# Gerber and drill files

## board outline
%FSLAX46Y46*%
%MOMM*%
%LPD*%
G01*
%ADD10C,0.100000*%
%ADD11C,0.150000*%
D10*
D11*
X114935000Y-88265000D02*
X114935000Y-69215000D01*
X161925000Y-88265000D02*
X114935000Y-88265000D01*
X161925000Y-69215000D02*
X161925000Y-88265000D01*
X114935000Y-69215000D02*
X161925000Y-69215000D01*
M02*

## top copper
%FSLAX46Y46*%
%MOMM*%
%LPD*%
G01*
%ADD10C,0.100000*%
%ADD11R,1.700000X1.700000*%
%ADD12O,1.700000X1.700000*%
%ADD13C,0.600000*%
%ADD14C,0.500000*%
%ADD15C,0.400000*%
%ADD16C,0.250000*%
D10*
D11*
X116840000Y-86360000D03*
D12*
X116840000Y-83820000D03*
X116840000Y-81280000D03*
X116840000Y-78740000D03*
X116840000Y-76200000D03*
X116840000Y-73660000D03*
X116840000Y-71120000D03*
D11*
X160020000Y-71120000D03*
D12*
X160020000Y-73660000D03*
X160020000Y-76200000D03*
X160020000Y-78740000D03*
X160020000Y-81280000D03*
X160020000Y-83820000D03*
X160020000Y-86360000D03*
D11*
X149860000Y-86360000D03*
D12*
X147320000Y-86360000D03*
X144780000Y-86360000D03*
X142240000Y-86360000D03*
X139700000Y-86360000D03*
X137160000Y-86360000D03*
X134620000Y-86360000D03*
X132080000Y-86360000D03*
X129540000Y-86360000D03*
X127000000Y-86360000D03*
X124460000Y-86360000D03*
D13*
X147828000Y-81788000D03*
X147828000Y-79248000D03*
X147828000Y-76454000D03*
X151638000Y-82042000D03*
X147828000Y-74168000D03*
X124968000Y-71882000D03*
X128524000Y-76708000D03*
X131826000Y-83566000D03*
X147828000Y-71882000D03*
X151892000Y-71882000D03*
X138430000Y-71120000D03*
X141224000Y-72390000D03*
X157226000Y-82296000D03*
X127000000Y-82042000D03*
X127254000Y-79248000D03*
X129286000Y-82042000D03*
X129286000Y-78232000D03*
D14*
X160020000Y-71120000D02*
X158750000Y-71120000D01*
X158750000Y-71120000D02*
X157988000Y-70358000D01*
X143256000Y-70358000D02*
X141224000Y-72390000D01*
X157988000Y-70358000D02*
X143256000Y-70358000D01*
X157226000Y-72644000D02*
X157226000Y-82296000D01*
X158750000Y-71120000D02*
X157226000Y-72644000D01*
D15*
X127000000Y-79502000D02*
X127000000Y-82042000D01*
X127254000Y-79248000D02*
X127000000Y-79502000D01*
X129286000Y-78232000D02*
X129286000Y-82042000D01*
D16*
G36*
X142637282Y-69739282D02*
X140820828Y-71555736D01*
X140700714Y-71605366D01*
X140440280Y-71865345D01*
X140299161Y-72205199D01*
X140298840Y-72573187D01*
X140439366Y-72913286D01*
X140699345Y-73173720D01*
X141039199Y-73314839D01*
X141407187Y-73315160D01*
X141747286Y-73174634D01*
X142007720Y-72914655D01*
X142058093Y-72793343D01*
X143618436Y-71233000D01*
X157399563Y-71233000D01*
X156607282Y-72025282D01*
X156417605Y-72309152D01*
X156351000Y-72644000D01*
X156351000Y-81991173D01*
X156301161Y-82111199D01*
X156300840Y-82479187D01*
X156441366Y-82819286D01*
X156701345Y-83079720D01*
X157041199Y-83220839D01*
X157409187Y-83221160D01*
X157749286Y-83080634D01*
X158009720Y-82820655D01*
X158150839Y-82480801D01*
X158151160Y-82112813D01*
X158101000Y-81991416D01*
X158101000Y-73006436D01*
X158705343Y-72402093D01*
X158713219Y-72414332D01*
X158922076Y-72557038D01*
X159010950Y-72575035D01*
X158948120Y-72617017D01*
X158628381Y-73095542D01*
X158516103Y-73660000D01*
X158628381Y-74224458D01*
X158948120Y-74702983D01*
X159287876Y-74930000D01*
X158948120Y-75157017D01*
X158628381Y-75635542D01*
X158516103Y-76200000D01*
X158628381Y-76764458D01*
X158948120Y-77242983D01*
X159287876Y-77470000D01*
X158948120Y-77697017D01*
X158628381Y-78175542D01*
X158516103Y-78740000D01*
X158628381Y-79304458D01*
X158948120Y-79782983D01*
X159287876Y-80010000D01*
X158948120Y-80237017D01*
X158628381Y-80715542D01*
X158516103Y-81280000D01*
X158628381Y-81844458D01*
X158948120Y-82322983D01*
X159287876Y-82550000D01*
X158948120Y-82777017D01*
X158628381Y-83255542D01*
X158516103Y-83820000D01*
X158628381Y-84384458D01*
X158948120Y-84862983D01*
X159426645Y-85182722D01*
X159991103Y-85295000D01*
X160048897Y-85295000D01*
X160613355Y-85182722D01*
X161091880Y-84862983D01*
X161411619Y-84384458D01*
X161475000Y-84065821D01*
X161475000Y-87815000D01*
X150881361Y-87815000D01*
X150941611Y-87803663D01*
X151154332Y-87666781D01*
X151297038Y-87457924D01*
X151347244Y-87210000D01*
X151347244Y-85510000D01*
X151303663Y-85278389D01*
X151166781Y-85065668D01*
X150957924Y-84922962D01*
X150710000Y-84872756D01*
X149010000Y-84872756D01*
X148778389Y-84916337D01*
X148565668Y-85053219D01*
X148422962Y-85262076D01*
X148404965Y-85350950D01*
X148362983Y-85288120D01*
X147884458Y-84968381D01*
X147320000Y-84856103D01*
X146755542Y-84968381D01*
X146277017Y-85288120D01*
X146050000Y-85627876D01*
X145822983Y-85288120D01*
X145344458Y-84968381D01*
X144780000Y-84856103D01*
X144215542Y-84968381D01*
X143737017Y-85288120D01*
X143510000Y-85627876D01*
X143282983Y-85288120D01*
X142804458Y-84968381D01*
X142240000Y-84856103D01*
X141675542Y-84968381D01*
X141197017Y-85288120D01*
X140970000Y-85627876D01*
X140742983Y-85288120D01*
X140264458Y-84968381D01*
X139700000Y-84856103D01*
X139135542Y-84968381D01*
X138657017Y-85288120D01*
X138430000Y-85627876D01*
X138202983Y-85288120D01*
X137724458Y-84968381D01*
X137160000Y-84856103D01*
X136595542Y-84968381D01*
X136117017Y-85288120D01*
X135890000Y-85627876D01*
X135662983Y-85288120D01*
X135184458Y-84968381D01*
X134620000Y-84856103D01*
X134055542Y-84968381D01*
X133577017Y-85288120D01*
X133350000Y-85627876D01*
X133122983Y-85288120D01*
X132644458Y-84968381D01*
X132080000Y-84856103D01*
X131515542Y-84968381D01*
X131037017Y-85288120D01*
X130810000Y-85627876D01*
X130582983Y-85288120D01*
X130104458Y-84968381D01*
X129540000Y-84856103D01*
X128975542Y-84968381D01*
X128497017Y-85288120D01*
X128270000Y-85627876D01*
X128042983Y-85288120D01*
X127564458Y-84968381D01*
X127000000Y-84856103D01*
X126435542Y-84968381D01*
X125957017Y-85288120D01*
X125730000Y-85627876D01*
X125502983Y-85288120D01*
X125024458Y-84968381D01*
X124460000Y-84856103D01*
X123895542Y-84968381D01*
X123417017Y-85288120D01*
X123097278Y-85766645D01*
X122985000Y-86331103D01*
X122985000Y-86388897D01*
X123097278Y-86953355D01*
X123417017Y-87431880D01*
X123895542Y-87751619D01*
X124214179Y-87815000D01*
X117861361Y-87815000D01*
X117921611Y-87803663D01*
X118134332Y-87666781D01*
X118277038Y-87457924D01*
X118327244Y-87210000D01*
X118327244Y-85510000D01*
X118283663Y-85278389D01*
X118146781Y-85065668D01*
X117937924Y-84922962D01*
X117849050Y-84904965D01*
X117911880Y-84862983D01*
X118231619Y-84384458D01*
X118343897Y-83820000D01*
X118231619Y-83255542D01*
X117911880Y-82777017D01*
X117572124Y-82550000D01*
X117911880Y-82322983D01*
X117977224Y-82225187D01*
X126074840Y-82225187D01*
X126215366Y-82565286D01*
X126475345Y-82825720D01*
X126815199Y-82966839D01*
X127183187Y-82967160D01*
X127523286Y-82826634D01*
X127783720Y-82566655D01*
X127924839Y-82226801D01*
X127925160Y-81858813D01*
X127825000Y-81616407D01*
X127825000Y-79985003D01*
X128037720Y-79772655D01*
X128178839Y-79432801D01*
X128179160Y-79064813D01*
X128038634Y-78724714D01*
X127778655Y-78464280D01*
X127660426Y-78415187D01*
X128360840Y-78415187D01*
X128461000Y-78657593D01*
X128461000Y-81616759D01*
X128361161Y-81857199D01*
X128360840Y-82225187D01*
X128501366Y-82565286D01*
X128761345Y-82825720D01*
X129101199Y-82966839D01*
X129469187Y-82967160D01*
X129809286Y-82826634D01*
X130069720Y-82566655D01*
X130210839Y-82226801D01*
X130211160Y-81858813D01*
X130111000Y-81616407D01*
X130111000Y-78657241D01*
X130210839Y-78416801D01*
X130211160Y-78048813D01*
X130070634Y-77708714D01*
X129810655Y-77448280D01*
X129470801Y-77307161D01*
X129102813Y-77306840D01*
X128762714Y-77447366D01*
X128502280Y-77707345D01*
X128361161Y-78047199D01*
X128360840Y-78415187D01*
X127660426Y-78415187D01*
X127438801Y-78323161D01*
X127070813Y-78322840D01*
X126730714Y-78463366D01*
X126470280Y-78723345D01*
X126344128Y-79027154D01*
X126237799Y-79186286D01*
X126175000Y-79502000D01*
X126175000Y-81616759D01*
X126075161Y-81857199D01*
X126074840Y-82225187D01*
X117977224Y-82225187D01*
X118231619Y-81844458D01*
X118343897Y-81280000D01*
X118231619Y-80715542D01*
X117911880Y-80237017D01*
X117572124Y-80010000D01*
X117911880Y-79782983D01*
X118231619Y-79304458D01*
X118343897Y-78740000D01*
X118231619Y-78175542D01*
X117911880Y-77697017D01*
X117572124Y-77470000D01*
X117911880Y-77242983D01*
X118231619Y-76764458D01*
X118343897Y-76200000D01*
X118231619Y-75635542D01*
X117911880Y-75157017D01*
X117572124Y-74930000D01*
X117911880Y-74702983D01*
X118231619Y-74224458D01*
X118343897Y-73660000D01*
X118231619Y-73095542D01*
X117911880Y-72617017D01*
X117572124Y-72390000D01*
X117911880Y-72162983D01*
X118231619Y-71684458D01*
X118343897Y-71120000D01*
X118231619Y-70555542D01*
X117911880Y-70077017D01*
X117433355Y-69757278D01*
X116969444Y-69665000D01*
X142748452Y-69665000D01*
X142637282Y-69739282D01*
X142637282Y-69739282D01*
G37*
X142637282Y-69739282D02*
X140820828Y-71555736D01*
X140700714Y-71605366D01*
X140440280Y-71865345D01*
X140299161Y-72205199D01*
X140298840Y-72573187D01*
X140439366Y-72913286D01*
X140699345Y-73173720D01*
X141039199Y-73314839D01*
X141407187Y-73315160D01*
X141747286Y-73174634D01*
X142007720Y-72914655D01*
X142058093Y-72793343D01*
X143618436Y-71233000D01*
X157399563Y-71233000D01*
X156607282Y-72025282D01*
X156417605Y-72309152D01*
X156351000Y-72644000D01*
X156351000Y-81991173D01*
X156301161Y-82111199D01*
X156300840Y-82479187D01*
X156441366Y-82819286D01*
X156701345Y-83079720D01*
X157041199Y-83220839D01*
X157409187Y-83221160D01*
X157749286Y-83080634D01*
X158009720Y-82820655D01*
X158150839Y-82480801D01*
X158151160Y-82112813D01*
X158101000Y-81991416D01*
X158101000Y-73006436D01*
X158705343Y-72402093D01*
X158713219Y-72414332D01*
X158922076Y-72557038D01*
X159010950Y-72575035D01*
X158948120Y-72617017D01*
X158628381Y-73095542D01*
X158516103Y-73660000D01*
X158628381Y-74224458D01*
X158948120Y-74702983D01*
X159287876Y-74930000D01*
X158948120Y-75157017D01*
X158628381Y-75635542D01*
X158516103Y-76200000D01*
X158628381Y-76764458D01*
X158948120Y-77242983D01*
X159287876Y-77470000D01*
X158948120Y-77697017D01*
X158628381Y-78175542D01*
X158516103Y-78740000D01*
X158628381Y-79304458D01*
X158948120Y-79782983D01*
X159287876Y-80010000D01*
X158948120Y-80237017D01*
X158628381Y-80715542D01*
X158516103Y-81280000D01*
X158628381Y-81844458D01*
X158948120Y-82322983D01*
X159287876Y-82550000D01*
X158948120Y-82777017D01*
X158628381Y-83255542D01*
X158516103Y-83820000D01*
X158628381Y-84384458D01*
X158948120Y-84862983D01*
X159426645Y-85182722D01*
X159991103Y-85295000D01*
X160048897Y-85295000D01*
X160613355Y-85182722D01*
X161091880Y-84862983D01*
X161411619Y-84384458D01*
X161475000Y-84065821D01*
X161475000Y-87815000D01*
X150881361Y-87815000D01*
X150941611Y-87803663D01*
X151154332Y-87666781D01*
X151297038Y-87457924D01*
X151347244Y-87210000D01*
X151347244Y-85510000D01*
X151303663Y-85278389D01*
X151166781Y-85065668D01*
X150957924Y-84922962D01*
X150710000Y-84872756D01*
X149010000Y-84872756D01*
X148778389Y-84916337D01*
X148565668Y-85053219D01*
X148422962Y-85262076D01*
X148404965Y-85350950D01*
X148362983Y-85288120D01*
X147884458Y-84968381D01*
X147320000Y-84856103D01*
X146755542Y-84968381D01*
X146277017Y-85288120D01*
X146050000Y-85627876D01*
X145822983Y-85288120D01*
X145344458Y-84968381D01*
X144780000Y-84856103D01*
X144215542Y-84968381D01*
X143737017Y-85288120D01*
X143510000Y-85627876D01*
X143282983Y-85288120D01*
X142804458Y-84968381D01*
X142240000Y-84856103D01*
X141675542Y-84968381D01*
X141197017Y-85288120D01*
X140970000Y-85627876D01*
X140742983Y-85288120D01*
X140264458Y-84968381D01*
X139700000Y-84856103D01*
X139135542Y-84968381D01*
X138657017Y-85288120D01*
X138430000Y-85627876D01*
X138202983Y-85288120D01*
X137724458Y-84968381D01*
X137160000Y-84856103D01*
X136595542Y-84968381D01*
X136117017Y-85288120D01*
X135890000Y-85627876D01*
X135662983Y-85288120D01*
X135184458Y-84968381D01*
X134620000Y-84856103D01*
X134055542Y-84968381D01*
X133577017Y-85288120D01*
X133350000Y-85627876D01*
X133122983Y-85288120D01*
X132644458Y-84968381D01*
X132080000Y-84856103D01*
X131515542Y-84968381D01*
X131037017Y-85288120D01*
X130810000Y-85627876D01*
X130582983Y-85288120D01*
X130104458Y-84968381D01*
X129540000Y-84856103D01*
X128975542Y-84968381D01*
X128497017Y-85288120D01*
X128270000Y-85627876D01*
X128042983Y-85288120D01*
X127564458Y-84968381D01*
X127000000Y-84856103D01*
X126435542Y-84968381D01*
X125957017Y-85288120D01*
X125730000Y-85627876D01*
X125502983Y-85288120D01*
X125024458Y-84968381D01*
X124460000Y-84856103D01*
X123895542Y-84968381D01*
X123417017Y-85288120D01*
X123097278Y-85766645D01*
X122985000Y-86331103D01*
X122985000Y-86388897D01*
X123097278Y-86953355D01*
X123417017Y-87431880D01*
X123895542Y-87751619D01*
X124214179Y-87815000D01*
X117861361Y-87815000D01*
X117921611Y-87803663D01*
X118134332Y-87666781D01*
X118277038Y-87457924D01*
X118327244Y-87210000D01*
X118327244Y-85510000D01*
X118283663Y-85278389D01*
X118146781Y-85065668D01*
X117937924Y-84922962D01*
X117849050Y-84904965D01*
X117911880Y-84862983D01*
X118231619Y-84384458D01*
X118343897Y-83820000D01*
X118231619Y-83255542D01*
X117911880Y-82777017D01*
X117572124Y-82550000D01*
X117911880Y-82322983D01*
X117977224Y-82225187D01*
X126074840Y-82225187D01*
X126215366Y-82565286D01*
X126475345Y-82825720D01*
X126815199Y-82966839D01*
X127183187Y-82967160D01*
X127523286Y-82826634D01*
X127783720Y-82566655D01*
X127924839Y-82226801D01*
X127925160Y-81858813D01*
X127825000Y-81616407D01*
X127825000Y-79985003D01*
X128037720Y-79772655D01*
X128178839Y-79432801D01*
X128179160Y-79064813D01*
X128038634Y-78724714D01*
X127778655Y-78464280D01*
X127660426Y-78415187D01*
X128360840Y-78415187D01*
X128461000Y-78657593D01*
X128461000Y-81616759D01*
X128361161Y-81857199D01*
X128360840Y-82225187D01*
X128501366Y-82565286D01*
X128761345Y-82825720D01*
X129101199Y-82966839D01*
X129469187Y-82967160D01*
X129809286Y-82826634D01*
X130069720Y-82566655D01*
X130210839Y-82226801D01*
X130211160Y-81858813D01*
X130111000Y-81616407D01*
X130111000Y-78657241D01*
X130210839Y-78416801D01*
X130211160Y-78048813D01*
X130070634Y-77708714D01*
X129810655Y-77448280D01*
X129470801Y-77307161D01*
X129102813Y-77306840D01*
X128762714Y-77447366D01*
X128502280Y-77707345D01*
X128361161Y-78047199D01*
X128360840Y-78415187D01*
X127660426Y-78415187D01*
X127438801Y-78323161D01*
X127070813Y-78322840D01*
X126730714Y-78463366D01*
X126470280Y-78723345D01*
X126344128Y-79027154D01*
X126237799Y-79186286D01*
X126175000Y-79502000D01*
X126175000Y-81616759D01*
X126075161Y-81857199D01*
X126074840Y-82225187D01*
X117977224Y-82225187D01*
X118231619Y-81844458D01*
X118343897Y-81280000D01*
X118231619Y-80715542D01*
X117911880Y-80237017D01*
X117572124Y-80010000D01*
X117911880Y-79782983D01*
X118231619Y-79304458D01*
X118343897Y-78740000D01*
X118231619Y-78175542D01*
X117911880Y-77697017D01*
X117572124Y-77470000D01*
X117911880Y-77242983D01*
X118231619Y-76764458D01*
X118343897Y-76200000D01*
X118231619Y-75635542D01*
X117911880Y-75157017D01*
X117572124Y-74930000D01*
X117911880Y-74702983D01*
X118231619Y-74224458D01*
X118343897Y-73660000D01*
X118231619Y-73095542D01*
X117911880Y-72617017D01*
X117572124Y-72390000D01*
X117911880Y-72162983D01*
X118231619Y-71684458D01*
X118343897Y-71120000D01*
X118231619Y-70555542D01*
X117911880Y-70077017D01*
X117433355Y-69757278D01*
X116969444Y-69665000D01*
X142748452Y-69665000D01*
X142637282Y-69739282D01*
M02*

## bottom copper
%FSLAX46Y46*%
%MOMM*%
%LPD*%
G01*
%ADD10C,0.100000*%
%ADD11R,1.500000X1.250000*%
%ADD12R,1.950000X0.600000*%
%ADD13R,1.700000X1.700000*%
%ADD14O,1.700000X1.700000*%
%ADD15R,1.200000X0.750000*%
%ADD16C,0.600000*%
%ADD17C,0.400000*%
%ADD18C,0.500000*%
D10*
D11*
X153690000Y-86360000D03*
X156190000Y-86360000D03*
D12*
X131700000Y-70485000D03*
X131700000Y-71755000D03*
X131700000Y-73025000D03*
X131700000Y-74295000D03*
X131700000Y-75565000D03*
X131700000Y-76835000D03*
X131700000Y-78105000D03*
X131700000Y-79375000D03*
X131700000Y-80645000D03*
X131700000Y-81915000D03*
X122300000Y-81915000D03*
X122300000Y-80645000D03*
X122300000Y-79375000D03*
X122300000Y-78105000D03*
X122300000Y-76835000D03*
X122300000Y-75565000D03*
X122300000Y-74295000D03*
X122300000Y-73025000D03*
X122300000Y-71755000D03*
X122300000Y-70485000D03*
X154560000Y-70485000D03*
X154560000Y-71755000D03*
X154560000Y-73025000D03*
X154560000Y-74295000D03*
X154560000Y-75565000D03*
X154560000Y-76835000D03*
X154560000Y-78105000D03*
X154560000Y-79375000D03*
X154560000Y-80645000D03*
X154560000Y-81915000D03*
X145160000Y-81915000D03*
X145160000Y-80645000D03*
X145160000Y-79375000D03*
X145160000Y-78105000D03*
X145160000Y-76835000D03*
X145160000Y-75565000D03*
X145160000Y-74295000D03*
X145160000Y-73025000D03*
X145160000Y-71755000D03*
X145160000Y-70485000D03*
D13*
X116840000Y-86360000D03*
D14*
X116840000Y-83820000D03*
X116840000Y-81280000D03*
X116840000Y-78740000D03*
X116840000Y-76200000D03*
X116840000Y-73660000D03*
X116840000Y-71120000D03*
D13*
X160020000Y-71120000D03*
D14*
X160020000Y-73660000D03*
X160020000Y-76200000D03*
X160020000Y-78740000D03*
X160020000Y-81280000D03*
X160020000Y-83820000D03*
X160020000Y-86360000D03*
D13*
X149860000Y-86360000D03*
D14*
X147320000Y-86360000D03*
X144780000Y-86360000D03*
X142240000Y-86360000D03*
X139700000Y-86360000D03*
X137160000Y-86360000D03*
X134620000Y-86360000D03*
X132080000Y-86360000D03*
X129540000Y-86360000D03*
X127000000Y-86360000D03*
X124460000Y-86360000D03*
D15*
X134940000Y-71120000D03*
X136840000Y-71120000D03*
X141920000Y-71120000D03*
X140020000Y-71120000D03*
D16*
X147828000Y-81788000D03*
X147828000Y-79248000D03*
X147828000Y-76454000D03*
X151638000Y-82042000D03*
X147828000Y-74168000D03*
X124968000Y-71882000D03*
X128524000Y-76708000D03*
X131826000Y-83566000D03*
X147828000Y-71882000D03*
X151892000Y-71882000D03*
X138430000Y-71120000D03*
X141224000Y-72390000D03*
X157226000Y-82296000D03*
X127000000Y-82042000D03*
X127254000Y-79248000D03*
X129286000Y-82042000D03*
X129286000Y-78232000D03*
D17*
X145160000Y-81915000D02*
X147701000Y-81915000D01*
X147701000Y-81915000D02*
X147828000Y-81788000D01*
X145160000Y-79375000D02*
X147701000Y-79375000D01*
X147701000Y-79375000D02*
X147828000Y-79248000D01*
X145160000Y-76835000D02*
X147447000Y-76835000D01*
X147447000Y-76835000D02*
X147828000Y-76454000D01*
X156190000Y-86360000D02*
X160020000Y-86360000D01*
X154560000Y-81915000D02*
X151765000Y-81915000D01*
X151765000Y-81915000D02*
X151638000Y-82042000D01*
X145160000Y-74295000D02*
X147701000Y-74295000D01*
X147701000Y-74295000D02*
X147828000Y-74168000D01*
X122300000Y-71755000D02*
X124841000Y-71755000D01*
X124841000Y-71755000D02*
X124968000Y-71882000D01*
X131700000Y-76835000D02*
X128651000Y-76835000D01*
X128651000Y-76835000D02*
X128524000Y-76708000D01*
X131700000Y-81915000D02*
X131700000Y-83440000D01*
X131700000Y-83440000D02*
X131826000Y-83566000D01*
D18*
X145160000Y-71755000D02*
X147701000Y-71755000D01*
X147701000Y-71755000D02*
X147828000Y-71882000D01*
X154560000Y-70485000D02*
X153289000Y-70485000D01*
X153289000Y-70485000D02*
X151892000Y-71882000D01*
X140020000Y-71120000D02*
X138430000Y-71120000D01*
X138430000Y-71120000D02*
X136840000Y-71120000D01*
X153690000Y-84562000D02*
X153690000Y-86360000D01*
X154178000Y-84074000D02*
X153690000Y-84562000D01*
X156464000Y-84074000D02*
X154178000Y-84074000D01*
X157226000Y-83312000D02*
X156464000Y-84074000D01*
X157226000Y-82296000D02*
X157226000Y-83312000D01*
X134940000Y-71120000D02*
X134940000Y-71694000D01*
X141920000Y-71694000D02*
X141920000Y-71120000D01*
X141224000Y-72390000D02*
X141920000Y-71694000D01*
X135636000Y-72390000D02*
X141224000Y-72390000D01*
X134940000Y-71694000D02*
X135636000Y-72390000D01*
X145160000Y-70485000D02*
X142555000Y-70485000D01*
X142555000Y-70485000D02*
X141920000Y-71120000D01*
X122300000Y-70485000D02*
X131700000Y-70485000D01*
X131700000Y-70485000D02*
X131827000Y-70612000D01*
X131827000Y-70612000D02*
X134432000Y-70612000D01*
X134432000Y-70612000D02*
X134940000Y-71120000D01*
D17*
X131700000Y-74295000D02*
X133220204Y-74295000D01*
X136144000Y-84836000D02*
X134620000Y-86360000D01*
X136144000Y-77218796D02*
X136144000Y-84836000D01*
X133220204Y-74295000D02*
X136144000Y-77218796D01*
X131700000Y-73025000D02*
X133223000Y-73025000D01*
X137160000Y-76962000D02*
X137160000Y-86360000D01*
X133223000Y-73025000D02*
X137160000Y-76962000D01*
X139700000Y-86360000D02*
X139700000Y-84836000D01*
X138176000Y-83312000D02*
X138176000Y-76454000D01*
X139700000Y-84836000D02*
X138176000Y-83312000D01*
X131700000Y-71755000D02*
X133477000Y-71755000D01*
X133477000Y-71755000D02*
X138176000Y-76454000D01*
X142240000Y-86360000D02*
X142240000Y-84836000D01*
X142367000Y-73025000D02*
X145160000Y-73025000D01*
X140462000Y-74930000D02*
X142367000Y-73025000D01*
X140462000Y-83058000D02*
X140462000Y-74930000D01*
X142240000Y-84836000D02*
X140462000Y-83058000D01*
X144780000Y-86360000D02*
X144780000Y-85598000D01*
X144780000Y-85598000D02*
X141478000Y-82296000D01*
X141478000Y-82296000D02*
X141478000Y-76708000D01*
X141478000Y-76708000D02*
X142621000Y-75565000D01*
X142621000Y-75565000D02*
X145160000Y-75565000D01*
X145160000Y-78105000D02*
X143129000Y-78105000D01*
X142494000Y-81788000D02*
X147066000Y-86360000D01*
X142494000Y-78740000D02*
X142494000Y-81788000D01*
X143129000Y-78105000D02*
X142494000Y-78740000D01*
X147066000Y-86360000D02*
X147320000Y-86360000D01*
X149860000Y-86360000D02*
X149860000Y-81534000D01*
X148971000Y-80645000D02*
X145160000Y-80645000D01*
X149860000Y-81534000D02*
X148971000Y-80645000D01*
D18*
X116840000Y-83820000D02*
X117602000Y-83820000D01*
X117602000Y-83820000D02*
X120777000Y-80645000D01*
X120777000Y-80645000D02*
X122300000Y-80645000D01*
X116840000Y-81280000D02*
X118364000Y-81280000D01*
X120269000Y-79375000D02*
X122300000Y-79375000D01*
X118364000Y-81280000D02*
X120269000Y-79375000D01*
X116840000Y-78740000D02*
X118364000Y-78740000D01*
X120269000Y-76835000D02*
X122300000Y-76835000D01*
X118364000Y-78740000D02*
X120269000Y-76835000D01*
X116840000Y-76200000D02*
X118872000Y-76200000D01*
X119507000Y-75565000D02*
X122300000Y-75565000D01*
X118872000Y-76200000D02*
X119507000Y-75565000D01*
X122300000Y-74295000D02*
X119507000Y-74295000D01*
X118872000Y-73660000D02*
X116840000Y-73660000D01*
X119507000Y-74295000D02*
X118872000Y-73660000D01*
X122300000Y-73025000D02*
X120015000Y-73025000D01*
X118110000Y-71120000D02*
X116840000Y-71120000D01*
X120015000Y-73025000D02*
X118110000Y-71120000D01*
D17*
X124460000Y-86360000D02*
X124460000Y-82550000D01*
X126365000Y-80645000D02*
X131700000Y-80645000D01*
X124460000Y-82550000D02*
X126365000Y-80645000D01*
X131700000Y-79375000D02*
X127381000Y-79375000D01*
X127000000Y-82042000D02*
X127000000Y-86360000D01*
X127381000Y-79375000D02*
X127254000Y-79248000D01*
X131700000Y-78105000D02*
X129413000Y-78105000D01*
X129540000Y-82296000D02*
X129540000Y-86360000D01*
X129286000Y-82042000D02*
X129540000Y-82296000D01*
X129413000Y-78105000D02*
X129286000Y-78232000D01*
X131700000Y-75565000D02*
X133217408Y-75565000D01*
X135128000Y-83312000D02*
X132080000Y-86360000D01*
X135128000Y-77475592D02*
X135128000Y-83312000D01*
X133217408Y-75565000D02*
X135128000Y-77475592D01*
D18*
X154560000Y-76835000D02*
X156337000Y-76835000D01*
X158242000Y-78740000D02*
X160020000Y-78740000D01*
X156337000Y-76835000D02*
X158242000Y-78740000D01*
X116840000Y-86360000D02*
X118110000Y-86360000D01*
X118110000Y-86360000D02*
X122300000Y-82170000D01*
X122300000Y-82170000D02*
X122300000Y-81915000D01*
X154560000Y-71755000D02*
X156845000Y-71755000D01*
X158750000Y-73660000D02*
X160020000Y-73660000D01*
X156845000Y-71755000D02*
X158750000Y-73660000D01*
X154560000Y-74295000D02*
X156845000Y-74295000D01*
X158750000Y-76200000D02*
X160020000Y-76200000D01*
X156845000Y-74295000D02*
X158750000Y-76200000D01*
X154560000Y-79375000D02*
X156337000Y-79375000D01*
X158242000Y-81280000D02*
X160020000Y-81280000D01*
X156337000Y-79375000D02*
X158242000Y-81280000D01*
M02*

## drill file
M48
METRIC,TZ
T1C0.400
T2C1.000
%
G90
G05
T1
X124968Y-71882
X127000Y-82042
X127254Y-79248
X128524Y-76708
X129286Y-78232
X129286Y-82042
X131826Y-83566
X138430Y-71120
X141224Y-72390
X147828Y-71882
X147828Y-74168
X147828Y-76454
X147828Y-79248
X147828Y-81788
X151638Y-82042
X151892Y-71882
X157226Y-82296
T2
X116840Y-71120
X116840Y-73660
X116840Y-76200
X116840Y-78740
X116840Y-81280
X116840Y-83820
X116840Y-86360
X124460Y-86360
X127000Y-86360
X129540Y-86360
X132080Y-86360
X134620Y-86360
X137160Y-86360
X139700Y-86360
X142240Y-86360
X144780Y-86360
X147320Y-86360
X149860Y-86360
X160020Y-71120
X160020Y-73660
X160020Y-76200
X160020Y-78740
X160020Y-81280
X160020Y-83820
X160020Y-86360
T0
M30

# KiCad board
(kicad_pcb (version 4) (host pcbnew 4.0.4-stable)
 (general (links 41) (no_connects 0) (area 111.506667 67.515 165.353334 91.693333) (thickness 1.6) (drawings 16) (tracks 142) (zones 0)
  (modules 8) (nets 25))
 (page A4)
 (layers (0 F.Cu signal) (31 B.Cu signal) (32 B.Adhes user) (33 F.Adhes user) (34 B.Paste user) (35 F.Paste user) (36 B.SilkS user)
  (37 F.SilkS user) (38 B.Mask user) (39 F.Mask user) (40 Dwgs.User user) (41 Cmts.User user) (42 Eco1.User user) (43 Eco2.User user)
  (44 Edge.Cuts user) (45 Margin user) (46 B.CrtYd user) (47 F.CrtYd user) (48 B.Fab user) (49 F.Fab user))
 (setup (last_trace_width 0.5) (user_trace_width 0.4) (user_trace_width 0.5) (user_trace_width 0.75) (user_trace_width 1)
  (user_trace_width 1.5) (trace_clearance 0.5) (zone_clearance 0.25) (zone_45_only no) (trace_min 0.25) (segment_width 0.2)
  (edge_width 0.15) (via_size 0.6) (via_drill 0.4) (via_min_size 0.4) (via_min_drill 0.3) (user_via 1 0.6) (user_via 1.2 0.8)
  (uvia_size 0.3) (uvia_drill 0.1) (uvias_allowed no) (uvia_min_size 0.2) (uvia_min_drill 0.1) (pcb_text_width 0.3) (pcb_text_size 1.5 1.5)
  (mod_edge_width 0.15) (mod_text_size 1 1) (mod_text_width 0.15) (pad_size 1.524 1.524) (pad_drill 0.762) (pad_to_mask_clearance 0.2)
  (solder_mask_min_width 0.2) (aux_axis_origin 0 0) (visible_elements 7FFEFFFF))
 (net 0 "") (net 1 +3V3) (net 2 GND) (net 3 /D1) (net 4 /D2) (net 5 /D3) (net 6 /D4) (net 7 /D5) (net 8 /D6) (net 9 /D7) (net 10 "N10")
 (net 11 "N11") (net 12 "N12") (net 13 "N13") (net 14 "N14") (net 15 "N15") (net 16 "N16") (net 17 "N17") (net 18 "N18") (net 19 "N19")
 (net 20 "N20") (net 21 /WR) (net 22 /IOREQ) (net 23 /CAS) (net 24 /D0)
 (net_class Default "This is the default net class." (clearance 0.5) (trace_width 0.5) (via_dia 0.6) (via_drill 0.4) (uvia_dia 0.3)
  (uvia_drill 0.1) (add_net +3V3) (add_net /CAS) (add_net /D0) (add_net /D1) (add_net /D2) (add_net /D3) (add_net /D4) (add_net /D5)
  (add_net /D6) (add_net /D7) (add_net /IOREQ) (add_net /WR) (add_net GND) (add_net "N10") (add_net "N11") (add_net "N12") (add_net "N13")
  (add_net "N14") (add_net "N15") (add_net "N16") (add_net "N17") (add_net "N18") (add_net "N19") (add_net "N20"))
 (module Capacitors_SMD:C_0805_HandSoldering (layer B.Cu) (at 154.94 86.36)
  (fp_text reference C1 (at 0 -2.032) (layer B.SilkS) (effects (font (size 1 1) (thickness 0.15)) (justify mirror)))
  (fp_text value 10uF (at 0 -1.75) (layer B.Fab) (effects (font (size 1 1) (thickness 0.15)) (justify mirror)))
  (pad 1 smd rect (at -1.25 0) (size 1.5 1.25) (layers B.Cu B.Paste B.Mask) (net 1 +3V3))
  (pad 2 smd rect (at 1.25 0) (size 1.5 1.25) (layers B.Cu B.Paste B.Mask) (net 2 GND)))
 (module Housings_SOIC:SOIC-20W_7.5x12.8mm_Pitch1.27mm (layer B.Cu) (at 127 76.2 180)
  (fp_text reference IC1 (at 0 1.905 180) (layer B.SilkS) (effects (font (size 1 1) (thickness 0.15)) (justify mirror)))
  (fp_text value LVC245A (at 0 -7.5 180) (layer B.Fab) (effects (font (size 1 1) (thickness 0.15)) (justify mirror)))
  (pad 1 smd rect (at -4.7 5.715 180) (size 1.95 0.6) (layers B.Cu B.Paste B.Mask) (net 1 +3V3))
  (pad 2 smd rect (at -4.7 4.445 180) (size 1.95 0.6) (layers B.Cu B.Paste B.Mask) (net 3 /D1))
  (pad 3 smd rect (at -4.7 3.175 180) (size 1.95 0.6) (layers B.Cu B.Paste B.Mask) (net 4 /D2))
  (pad 4 smd rect (at -4.7 1.905 180) (size 1.95 0.6) (layers B.Cu B.Paste B.Mask) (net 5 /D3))
  (pad 5 smd rect (at -4.7 0.635 180) (size 1.95 0.6) (layers B.Cu B.Paste B.Mask) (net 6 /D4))
  (pad 6 smd rect (at -4.7 -0.635 180) (size 1.95 0.6) (layers B.Cu B.Paste B.Mask) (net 2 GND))
  (pad 7 smd rect (at -4.7 -1.905 180) (size 1.95 0.6) (layers B.Cu B.Paste B.Mask) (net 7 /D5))
  (pad 8 smd rect (at -4.7 -3.175 180) (size 1.95 0.6) (layers B.Cu B.Paste B.Mask) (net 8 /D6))
  (pad 9 smd rect (at -4.7 -4.445 180) (size 1.95 0.6) (layers B.Cu B.Paste B.Mask) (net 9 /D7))
  (pad 10 smd rect (at -4.7 -5.715 180) (size 1.95 0.6) (layers B.Cu B.Paste B.Mask) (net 2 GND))
  (pad 11 smd rect (at 4.7 -5.715 180) (size 1.95 0.6) (layers B.Cu B.Paste B.Mask) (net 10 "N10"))
  (pad 12 smd rect (at 4.7 -4.445 180) (size 1.95 0.6) (layers B.Cu B.Paste B.Mask) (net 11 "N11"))
  (pad 13 smd rect (at 4.7 -3.175 180) (size 1.95 0.6) (layers B.Cu B.Paste B.Mask) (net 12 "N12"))
  (pad 14 smd rect (at 4.7 -1.905 180) (size 1.95 0.6) (layers B.Cu B.Paste B.Mask))
  (pad 15 smd rect (at 4.7 -0.635 180) (size 1.95 0.6) (layers B.Cu B.Paste B.Mask) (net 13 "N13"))
  (pad 16 smd rect (at 4.7 0.635 180) (size 1.95 0.6) (layers B.Cu B.Paste B.Mask) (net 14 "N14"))
  (pad 17 smd rect (at 4.7 1.905 180) (size 1.95 0.6) (layers B.Cu B.Paste B.Mask) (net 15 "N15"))
  (pad 18 smd rect (at 4.7 3.175 180) (size 1.95 0.6) (layers B.Cu B.Paste B.Mask) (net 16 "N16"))
  (pad 19 smd rect (at 4.7 4.445 180) (size 1.95 0.6) (layers B.Cu B.Paste B.Mask) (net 2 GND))
  (pad 20 smd rect (at 4.7 5.715 180) (size 1.95 0.6) (layers B.Cu B.Paste B.Mask) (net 1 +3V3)))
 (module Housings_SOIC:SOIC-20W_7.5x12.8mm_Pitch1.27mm (layer B.Cu) (at 149.86 76.2 180)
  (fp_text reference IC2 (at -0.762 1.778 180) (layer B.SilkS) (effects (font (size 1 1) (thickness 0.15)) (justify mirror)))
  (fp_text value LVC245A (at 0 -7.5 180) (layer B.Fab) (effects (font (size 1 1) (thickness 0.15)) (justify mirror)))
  (pad 1 smd rect (at -4.7 5.715 180) (size 1.95 0.6) (layers B.Cu B.Paste B.Mask) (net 2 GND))
  (pad 2 smd rect (at -4.7 4.445 180) (size 1.95 0.6) (layers B.Cu B.Paste B.Mask) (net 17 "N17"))
  (pad 3 smd rect (at -4.7 3.175 180) (size 1.95 0.6) (layers B.Cu B.Paste B.Mask))
  (pad 4 smd rect (at -4.7 1.905 180) (size 1.95 0.6) (layers B.Cu B.Paste B.Mask) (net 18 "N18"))
  (pad 5 smd rect (at -4.7 0.635 180) (size 1.95 0.6) (layers B.Cu B.Paste B.Mask))
  (pad 6 smd rect (at -4.7 -0.635 180) (size 1.95 0.6) (layers B.Cu B.Paste B.Mask) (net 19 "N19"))
  (pad 7 smd rect (at -4.7 -1.905 180) (size 1.95 0.6) (layers B.Cu B.Paste B.Mask))
  (pad 8 smd rect (at -4.7 -3.175 180) (size 1.95 0.6) (layers B.Cu B.Paste B.Mask) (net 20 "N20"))
  (pad 9 smd rect (at -4.7 -4.445 180) (size 1.95 0.6) (layers B.Cu B.Paste B.Mask))
  (pad 10 smd rect (at -4.7 -5.715 180) (size 1.95 0.6) (layers B.Cu B.Paste B.Mask) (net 2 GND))
  (pad 11 smd rect (at 4.7 -5.715 180) (size 1.95 0.6) (layers B.Cu B.Paste B.Mask) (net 2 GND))
  (pad 12 smd rect (at 4.7 -4.445 180) (size 1.95 0.6) (layers B.Cu B.Paste B.Mask) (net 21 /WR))
  (pad 13 smd rect (at 4.7 -3.175 180) (size 1.95 0.6) (layers B.Cu B.Paste B.Mask) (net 2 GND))
  (pad 14 smd rect (at 4.7 -1.905 180) (size 1.95 0.6) (layers B.Cu B.Paste B.Mask) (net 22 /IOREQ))
  (pad 15 smd rect (at 4.7 -0.635 180) (size 1.95 0.6) (layers B.Cu B.Paste B.Mask) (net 2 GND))
  (pad 16 smd rect (at 4.7 0.635 180) (size 1.95 0.6) (layers B.Cu B.Paste B.Mask) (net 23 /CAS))
  (pad 17 smd rect (at 4.7 1.905 180) (size 1.95 0.6) (layers B.Cu B.Paste B.Mask) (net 2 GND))
  (pad 18 smd rect (at 4.7 3.175 180) (size 1.95 0.6) (layers B.Cu B.Paste B.Mask) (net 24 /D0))
  (pad 19 smd rect (at 4.7 4.445 180) (size 1.95 0.6) (layers B.Cu B.Paste B.Mask) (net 2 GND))
  (pad 20 smd rect (at 4.7 5.715 180) (size 1.95 0.6) (layers B.Cu B.Paste B.Mask) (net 1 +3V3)))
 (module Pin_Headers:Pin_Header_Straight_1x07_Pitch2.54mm (layer F.Cu) (at 116.84 86.36 180)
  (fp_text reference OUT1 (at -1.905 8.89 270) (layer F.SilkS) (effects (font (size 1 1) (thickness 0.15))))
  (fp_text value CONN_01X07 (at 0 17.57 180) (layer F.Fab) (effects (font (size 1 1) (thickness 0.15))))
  (pad 1 thru_hole rect (at 0 0 180) (size 1.7 1.7) (drill 1) (layers *.Cu *.Mask) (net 10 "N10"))
  (pad 2 thru_hole oval (at 0 2.54 180) (size 1.7 1.7) (drill 1) (layers *.Cu *.Mask) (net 11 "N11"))
  (pad 3 thru_hole oval (at 0 5.08 180) (size 1.7 1.7) (drill 1) (layers *.Cu *.Mask) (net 12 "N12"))
  (pad 4 thru_hole oval (at 0 7.62 180) (size 1.7 1.7) (drill 1) (layers *.Cu *.Mask) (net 13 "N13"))
  (pad 5 thru_hole oval (at 0 10.16 180) (size 1.7 1.7) (drill 1) (layers *.Cu *.Mask) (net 14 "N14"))
  (pad 6 thru_hole oval (at 0 12.7 180) (size 1.7 1.7) (drill 1) (layers *.Cu *.Mask) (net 15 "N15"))
  (pad 7 thru_hole oval (at 0 15.24 180) (size 1.7 1.7) (drill 1) (layers *.Cu *.Mask) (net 16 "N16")))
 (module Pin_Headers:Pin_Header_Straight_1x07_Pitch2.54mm (layer F.Cu) (at 160.02 71.12)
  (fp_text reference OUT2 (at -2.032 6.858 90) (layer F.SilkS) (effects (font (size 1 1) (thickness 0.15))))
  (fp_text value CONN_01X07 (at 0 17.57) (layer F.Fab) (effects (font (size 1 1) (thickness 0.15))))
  (pad 1 thru_hole rect (at 0 0) (size 1.7 1.7) (drill 1) (layers *.Cu *.Mask) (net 1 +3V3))
  (pad 2 thru_hole oval (at 0 2.54) (size 1.7 1.7) (drill 1) (layers *.Cu *.Mask) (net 17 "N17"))
  (pad 3 thru_hole oval (at 0 5.08) (size 1.7 1.7) (drill 1) (layers *.Cu *.Mask) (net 18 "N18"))
  (pad 4 thru_hole oval (at 0 7.62) (size 1.7 1.7) (drill 1) (layers *.Cu *.Mask) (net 19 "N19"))
  (pad 5 thru_hole oval (at 0 10.16) (size 1.7 1.7) (drill 1) (layers *.Cu *.Mask) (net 20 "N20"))
  (pad 6 thru_hole oval (at 0 12.7) (size 1.7 1.7) (drill 1) (layers *.Cu *.Mask))
  (pad 7 thru_hole oval (at 0 15.24) (size 1.7 1.7) (drill 1) (layers *.Cu *.Mask) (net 2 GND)))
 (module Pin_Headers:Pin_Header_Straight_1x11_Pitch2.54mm (layer F.Cu) (at 149.86 86.36 270)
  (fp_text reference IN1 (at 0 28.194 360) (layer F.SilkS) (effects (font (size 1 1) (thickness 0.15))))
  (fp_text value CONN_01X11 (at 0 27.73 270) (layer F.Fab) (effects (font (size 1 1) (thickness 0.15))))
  (pad 1 thru_hole rect (at 0 0 270) (size 1.7 1.7) (drill 1) (layers *.Cu *.Mask) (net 21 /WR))
  (pad 2 thru_hole oval (at 0 2.54 270) (size 1.7 1.7) (drill 1) (layers *.Cu *.Mask) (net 22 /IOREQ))
  (pad 3 thru_hole oval (at 0 5.08 270) (size 1.7 1.7) (drill 1) (layers *.Cu *.Mask) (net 23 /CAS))
  (pad 4 thru_hole oval (at 0 7.62 270) (size 1.7 1.7) (drill 1) (layers *.Cu *.Mask) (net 24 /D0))
  (pad 5 thru_hole oval (at 0 10.16 270) (size 1.7 1.7) (drill 1) (layers *.Cu *.Mask) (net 3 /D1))
  (pad 6 thru_hole oval (at 0 12.7 270) (size 1.7 1.7) (drill 1) (layers *.Cu *.Mask) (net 4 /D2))
  (pad 7 thru_hole oval (at 0 15.24 270) (size 1.7 1.7) (drill 1) (layers *.Cu *.Mask) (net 5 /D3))
  (pad 8 thru_hole oval (at 0 17.78 270) (size 1.7 1.7) (drill 1) (layers *.Cu *.Mask) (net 6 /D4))
  (pad 9 thru_hole oval (at 0 20.32 270) (size 1.7 1.7) (drill 1) (layers *.Cu *.Mask) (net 7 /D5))
  (pad 10 thru_hole oval (at 0 22.86 270) (size 1.7 1.7) (drill 1) (layers *.Cu *.Mask) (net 8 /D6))
  (pad 11 thru_hole oval (at 0 25.4 270) (size 1.7 1.7) (drill 1) (layers *.Cu *.Mask) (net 9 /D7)))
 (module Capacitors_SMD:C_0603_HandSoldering (layer B.Cu) (at 135.89 71.12)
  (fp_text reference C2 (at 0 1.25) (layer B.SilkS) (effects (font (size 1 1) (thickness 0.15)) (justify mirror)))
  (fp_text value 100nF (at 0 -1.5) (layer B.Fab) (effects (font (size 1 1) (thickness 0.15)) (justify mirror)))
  (pad 1 smd rect (at -0.95 0) (size 1.2 0.75) (layers B.Cu B.Paste B.Mask) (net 1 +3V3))
  (pad 2 smd rect (at 0.95 0) (size 1.2 0.75) (layers B.Cu B.Paste B.Mask) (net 2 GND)))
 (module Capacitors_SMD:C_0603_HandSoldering (layer B.Cu) (at 140.97 71.12 180)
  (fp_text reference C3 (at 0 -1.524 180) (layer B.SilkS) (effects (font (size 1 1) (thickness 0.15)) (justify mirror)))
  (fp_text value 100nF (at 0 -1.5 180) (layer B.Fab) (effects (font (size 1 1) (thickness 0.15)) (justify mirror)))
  (pad 1 smd rect (at -0.95 0 180) (size 1.2 0.75) (layers B.Cu B.Paste B.Mask) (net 1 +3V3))
  (pad 2 smd rect (at 0.95 0 180) (size 1.2 0.75) (layers B.Cu B.Paste B.Mask) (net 2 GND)))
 (gr_line (start 114.935 88.265) (end 114.935 69.215) (angle 90) (layer Edge.Cuts) (width 0.15))
 (gr_line (start 161.925 88.265) (end 114.935 88.265) (angle 90) (layer Edge.Cuts) (width 0.15))
 (gr_line (start 161.925 69.215) (end 161.925 88.265) (angle 90) (layer Edge.Cuts) (width 0.15))
 (gr_line (start 114.935 69.215) (end 161.925 69.215) (angle 90) (layer Edge.Cuts) (width 0.15))
 (segment (start 145.16 81.915) (end 147.701 81.915) (width 0.4) (layer B.Cu) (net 2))
 (via (at 147.828 81.788) (size 0.6) (drill 0.4) (layers F.Cu B.Cu) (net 2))
 (segment (start 147.701 81.915) (end 147.828 81.788) (width 0.4) (layer B.Cu) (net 2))
 (segment (start 145.16 79.375) (end 147.701 79.375) (width 0.4) (layer B.Cu) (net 2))
 (via (at 147.828 79.248) (size 0.6) (drill 0.4) (layers F.Cu B.Cu) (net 2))
 (segment (start 147.701 79.375) (end 147.828 79.248) (width 0.4) (layer B.Cu) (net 2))
 (segment (start 145.16 76.835) (end 147.447 76.835) (width 0.4) (layer B.Cu) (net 2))
 (via (at 147.828 76.454) (size 0.6) (drill 0.4) (layers F.Cu B.Cu) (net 2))
 (segment (start 147.447 76.835) (end 147.828 76.454) (width 0.4) (layer B.Cu) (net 2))
 (segment (start 156.19 86.36) (end 160.02 86.36) (width 0.4) (layer B.Cu) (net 2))
 (segment (start 154.56 81.915) (end 151.765 81.915) (width 0.4) (layer B.Cu) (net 2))
 (via (at 151.638 82.042) (size 0.6) (drill 0.4) (layers F.Cu B.Cu) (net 2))
 (segment (start 151.765 81.915) (end 151.638 82.042) (width 0.4) (layer B.Cu) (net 2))
 (segment (start 145.16 74.295) (end 147.701 74.295) (width 0.4) (layer B.Cu) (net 2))
 (via (at 147.828 74.168) (size 0.6) (drill 0.4) (layers F.Cu B.Cu) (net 2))
 (segment (start 147.701 74.295) (end 147.828 74.168) (width 0.4) (layer B.Cu) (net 2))
 (segment (start 122.3 71.755) (end 124.841 71.755) (width 0.4) (layer B.Cu) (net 2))
 (via (at 124.968 71.882) (size 0.6) (drill 0.4) (layers F.Cu B.Cu) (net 2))
 (segment (start 124.841 71.755) (end 124.968 71.882) (width 0.4) (layer B.Cu) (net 2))
 (segment (start 131.7 76.835) (end 128.651 76.835) (width 0.4) (layer B.Cu) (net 2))
 (via (at 128.524 76.708) (size 0.6) (drill 0.4) (layers F.Cu B.Cu) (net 2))
 (segment (start 128.651 76.835) (end 128.524 76.708) (width 0.4) (layer B.Cu) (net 2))
 (segment (start 131.7 81.915) (end 131.7 83.44) (width 0.4) (layer B.Cu) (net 2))
 (via (at 131.826 83.566) (size 0.6) (drill 0.4) (layers F.Cu B.Cu) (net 2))
 (segment (start 131.7 83.44) (end 131.826 83.566) (width 0.4) (layer B.Cu) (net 2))
 (segment (start 145.16 71.755) (end 147.701 71.755) (width 0.5) (layer B.Cu) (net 2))
 (via (at 147.828 71.882) (size 0.6) (drill 0.4) (layers F.Cu B.Cu) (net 2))
 (segment (start 147.701 71.755) (end 147.828 71.882) (width 0.5) (layer B.Cu) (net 2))
 (segment (start 154.56 70.485) (end 153.289 70.485) (width 0.5) (layer B.Cu) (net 2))
 (via (at 151.892 71.882) (size 0.6) (drill 0.4) (layers F.Cu B.Cu) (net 2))
 (segment (start 153.289 70.485) (end 151.892 71.882) (width 0.5) (layer B.Cu) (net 2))
 (segment (start 140.02 71.12) (end 138.43 71.12) (width 0.5) (layer B.Cu) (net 2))
 (via (at 138.43 71.12) (size 0.6) (drill 0.4) (layers F.Cu B.Cu) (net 2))
 (segment (start 138.43 71.12) (end 136.84 71.12) (width 0.5) (layer B.Cu) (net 2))
 (segment (start 160.02 71.12) (end 158.75 71.12) (width 0.5) (layer F.Cu) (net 1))
 (segment (start 158.75 71.12) (end 157.988 70.358) (width 0.5) (layer F.Cu) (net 1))
 (via (at 141.224 72.39) (size 0.6) (drill 0.4) (layers F.Cu B.Cu) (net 1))
 (segment (start 143.256 70.358) (end 141.224 72.39) (width 0.5) (layer F.Cu) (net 1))
 (segment (start 157.988 70.358) (end 143.256 70.358) (width 0.5) (layer F.Cu) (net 1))
 (segment (start 153.69 84.562) (end 153.69 86.36) (width 0.5) (layer B.Cu) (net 1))
 (segment (start 154.178 84.074) (end 153.69 84.562) (width 0.5) (layer B.Cu) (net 1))
 (segment (start 156.464 84.074) (end 154.178 84.074) (width 0.5) (layer B.Cu) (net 1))
 (segment (start 157.226 83.312) (end 156.464 84.074) (width 0.5) (layer B.Cu) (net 1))
 (segment (start 157.226 82.296) (end 157.226 83.312) (width 0.5) (layer B.Cu) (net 1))
 (via (at 157.226 82.296) (size 0.6) (drill 0.4) (layers F.Cu B.Cu) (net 1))
 (segment (start 157.226 72.644) (end 157.226 82.296) (width 0.5) (layer F.Cu) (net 1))
 (segment (start 158.75 71.12) (end 157.226 72.644) (width 0.5) (layer F.Cu) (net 1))
 (segment (start 134.94 71.12) (end 134.94 71.694) (width 0.5) (layer B.Cu) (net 1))
 (segment (start 141.92 71.694) (end 141.92 71.12) (width 0.5) (layer B.Cu) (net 1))
 (segment (start 141.224 72.39) (end 141.92 71.694) (width 0.5) (layer B.Cu) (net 1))
 (segment (start 135.636 72.39) (end 141.224 72.39) (width 0.5) (layer B.Cu) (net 1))
 (segment (start 134.94 71.694) (end 135.636 72.39) (width 0.5) (layer B.Cu) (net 1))
 (segment (start 145.16 70.485) (end 142.555 70.485) (width 0.5) (layer B.Cu) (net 1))
 (segment (start 142.555 70.485) (end 141.92 71.12) (width 0.5) (layer B.Cu) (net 1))
 (segment (start 122.3 70.485) (end 131.7 70.485) (width 0.5) (layer B.Cu) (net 1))
 (segment (start 131.7 70.485) (end 131.827 70.612) (width 0.5) (layer B.Cu) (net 1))
 (segment (start 131.827 70.612) (end 134.432 70.612) (width 0.5) (layer B.Cu) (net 1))
 (segment (start 134.432 70.612) (end 134.94 71.12) (width 0.5) (layer B.Cu) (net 1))
 (segment (start 131.7 74.295) (end 133.220204 74.295) (width 0.4) (layer B.Cu) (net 5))
 (segment (start 136.144 84.836) (end 134.62 86.36) (width 0.4) (layer B.Cu) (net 5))
 (segment (start 136.144 77.218796) (end 136.144 84.836) (width 0.4) (layer B.Cu) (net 5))
 (segment (start 133.220204 74.295) (end 136.144 77.218796) (width 0.4) (layer B.Cu) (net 5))
 (segment (start 131.7 73.025) (end 133.223 73.025) (width 0.4) (layer B.Cu) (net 4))
 (segment (start 137.16 76.962) (end 137.16 86.36) (width 0.4) (layer B.Cu) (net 4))
 (segment (start 133.223 73.025) (end 137.16 76.962) (width 0.4) (layer B.Cu) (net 4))
 (segment (start 139.7 86.36) (end 139.7 84.836) (width 0.4) (layer B.Cu) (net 3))
 (segment (start 138.176 83.312) (end 138.176 76.454) (width 0.4) (layer B.Cu) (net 3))
 (segment (start 139.7 84.836) (end 138.176 83.312) (width 0.4) (layer B.Cu) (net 3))
 (segment (start 131.7 71.755) (end 133.477 71.755) (width 0.4) (layer B.Cu) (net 3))
 (segment (start 133.477 71.755) (end 138.176 76.454) (width 0.4) (layer B.Cu) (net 3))
 (segment (start 142.24 86.36) (end 142.24 84.836) (width 0.4) (layer B.Cu) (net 24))
 (segment (start 142.367 73.025) (end 145.16 73.025) (width 0.4) (layer B.Cu) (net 24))
 (segment (start 140.462 74.93) (end 142.367 73.025) (width 0.4) (layer B.Cu) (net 24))
 (segment (start 140.462 83.058) (end 140.462 74.93) (width 0.4) (layer B.Cu) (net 24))
 (segment (start 142.24 84.836) (end 140.462 83.058) (width 0.4) (layer B.Cu) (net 24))
 (segment (start 144.78 86.36) (end 144.78 85.598) (width 0.4) (layer B.Cu) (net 23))
 (segment (start 144.78 85.598) (end 141.478 82.296) (width 0.4) (layer B.Cu) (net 23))
 (segment (start 141.478 82.296) (end 141.478 76.708) (width 0.4) (layer B.Cu) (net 23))
 (segment (start 141.478 76.708) (end 142.621 75.565) (width 0.4) (layer B.Cu) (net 23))
 (segment (start 142.621 75.565) (end 145.16 75.565) (width 0.4) (layer B.Cu) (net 23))
 (segment (start 145.16 78.105) (end 143.129 78.105) (width 0.4) (layer B.Cu) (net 22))
 (segment (start 142.494 81.788) (end 147.066 86.36) (width 0.4) (layer B.Cu) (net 22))
 (segment (start 142.494 78.74) (end 142.494 81.788) (width 0.4) (layer B.Cu) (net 22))
 (segment (start 143.129 78.105) (end 142.494 78.74) (width 0.4) (layer B.Cu) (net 22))
 (segment (start 147.066 86.36) (end 147.32 86.36) (width 0.4) (layer B.Cu) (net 22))
 (segment (start 149.86 86.36) (end 149.86 81.534) (width 0.4) (layer B.Cu) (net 21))
 (segment (start 148.971 80.645) (end 145.16 80.645) (width 0.4) (layer B.Cu) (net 21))
 (segment (start 149.86 81.534) (end 148.971 80.645) (width 0.4) (layer B.Cu) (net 21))
 (segment (start 116.84 83.82) (end 117.602 83.82) (width 0.5) (layer B.Cu) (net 11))
 (segment (start 117.602 83.82) (end 120.777 80.645) (width 0.5) (layer B.Cu) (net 11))
 (segment (start 120.777 80.645) (end 122.3 80.645) (width 0.5) (layer B.Cu) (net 11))
 (segment (start 116.84 81.28) (end 118.364 81.28) (width 0.5) (layer B.Cu) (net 12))
 (segment (start 120.269 79.375) (end 122.3 79.375) (width 0.5) (layer B.Cu) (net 12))
 (segment (start 118.364 81.28) (end 120.269 79.375) (width 0.5) (layer B.Cu) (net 12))
 (segment (start 116.84 78.74) (end 118.364 78.74) (width 0.5) (layer B.Cu) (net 13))
 (segment (start 120.269 76.835) (end 122.3 76.835) (width 0.5) (layer B.Cu) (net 13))
 (segment (start 118.364 78.74) (end 120.269 76.835) (width 0.5) (layer B.Cu) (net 13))
 (segment (start 116.84 76.2) (end 118.872 76.2) (width 0.5) (layer B.Cu) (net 14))
 (segment (start 119.507 75.565) (end 122.3 75.565) (width 0.5) (layer B.Cu) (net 14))
 (segment (start 118.872 76.2) (end 119.507 75.565) (width 0.5) (layer B.Cu) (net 14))
 (segment (start 122.3 74.295) (end 119.507 74.295) (width 0.5) (layer B.Cu) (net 15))
 (segment (start 118.872 73.66) (end 116.84 73.66) (width 0.5) (layer B.Cu) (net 15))
 (segment (start 119.507 74.295) (end 118.872 73.66) (width 0.5) (layer B.Cu) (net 15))
 (segment (start 122.3 73.025) (end 120.015 73.025) (width 0.5) (layer B.Cu) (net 16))
 (segment (start 118.11 71.12) (end 116.84 71.12) (width 0.5) (layer B.Cu) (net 16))
 (segment (start 120.015 73.025) (end 118.11 71.12) (width 0.5) (layer B.Cu) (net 16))
 (segment (start 124.46 86.36) (end 124.46 82.55) (width 0.4) (layer B.Cu) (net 9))
 (segment (start 126.365 80.645) (end 131.7 80.645) (width 0.4) (layer B.Cu) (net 9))
 (segment (start 124.46 82.55) (end 126.365 80.645) (width 0.4) (layer B.Cu) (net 9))
 (segment (start 131.7 79.375) (end 127.381 79.375) (width 0.4) (layer B.Cu) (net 8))
 (segment (start 127 82.042) (end 127 86.36) (width 0.4) (layer B.Cu) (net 8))
 (via (at 127 82.042) (size 0.6) (drill 0.4) (layers F.Cu B.Cu) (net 8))
 (segment (start 127 79.502) (end 127 82.042) (width 0.4) (layer F.Cu) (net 8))
 (segment (start 127.254 79.248) (end 127 79.502) (width 0.4) (layer F.Cu) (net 8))
 (via (at 127.254 79.248) (size 0.6) (drill 0.4) (layers F.Cu B.Cu) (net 8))
 (segment (start 127.381 79.375) (end 127.254 79.248) (width 0.4) (layer B.Cu) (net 8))
 (segment (start 131.7 78.105) (end 129.413 78.105) (width 0.4) (layer B.Cu) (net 7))
 (segment (start 129.54 82.296) (end 129.54 86.36) (width 0.4) (layer B.Cu) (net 7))
 (segment (start 129.286 82.042) (end 129.54 82.296) (width 0.4) (layer B.Cu) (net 7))
 (via (at 129.286 82.042) (size 0.6) (drill 0.4) (layers F.Cu B.Cu) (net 7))
 (segment (start 129.286 78.232) (end 129.286 82.042) (width 0.4) (layer F.Cu) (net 7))
 (via (at 129.286 78.232) (size 0.6) (drill 0.4) (layers F.Cu B.Cu) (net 7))
 (segment (start 129.413 78.105) (end 129.286 78.232) (width 0.4) (layer B.Cu) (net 7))
 (segment (start 131.7 75.565) (end 133.217408 75.565) (width 0.4) (layer B.Cu) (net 6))
 (segment (start 135.128 83.312) (end 132.08 86.36) (width 0.4) (layer B.Cu) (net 6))
 (segment (start 135.128 77.475592) (end 135.128 83.312) (width 0.4) (layer B.Cu) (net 6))
 (segment (start 133.217408 75.565) (end 135.128 77.475592) (width 0.4) (layer B.Cu) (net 6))
 (segment (start 154.56 76.835) (end 156.337 76.835) (width 0.5) (layer B.Cu) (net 19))
 (segment (start 158.242 78.74) (end 160.02 78.74) (width 0.5) (layer B.Cu) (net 19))
 (segment (start 156.337 76.835) (end 158.242 78.74) (width 0.5) (layer B.Cu) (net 19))
 (segment (start 116.84 86.36) (end 118.11 86.36) (width 0.5) (layer B.Cu) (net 10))
 (segment (start 118.11 86.36) (end 122.3 82.17) (width 0.5) (layer B.Cu) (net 10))
 (segment (start 122.3 82.17) (end 122.3 81.915) (width 0.5) (layer B.Cu) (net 10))
 (segment (start 154.56 71.755) (end 156.845 71.755) (width 0.5) (layer B.Cu) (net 17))
 (segment (start 158.75 73.66) (end 160.02 73.66) (width 0.5) (layer B.Cu) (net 17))
 (segment (start 156.845 71.755) (end 158.75 73.66) (width 0.5) (layer B.Cu) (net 17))
 (segment (start 154.56 74.295) (end 156.845 74.295) (width 0.5) (layer B.Cu) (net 18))
 (segment (start 158.75 76.2) (end 160.02 76.2) (width 0.5) (layer B.Cu) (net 18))
 (segment (start 156.845 74.295) (end 158.75 76.2) (width 0.5) (layer B.Cu) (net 18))
 (segment (start 154.56 79.375) (end 156.337 79.375) (width 0.5) (layer B.Cu) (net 20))
 (segment (start 158.242 81.28) (end 160.02 81.28) (width 0.5) (layer B.Cu) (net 20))
 (segment (start 156.337 79.375) (end 158.242 81.28) (width 0.5) (layer B.Cu) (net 20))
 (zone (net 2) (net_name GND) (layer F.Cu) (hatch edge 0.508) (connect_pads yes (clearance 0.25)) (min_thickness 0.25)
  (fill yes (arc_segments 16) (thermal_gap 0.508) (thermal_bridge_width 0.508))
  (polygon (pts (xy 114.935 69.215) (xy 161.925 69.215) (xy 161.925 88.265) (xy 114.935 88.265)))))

